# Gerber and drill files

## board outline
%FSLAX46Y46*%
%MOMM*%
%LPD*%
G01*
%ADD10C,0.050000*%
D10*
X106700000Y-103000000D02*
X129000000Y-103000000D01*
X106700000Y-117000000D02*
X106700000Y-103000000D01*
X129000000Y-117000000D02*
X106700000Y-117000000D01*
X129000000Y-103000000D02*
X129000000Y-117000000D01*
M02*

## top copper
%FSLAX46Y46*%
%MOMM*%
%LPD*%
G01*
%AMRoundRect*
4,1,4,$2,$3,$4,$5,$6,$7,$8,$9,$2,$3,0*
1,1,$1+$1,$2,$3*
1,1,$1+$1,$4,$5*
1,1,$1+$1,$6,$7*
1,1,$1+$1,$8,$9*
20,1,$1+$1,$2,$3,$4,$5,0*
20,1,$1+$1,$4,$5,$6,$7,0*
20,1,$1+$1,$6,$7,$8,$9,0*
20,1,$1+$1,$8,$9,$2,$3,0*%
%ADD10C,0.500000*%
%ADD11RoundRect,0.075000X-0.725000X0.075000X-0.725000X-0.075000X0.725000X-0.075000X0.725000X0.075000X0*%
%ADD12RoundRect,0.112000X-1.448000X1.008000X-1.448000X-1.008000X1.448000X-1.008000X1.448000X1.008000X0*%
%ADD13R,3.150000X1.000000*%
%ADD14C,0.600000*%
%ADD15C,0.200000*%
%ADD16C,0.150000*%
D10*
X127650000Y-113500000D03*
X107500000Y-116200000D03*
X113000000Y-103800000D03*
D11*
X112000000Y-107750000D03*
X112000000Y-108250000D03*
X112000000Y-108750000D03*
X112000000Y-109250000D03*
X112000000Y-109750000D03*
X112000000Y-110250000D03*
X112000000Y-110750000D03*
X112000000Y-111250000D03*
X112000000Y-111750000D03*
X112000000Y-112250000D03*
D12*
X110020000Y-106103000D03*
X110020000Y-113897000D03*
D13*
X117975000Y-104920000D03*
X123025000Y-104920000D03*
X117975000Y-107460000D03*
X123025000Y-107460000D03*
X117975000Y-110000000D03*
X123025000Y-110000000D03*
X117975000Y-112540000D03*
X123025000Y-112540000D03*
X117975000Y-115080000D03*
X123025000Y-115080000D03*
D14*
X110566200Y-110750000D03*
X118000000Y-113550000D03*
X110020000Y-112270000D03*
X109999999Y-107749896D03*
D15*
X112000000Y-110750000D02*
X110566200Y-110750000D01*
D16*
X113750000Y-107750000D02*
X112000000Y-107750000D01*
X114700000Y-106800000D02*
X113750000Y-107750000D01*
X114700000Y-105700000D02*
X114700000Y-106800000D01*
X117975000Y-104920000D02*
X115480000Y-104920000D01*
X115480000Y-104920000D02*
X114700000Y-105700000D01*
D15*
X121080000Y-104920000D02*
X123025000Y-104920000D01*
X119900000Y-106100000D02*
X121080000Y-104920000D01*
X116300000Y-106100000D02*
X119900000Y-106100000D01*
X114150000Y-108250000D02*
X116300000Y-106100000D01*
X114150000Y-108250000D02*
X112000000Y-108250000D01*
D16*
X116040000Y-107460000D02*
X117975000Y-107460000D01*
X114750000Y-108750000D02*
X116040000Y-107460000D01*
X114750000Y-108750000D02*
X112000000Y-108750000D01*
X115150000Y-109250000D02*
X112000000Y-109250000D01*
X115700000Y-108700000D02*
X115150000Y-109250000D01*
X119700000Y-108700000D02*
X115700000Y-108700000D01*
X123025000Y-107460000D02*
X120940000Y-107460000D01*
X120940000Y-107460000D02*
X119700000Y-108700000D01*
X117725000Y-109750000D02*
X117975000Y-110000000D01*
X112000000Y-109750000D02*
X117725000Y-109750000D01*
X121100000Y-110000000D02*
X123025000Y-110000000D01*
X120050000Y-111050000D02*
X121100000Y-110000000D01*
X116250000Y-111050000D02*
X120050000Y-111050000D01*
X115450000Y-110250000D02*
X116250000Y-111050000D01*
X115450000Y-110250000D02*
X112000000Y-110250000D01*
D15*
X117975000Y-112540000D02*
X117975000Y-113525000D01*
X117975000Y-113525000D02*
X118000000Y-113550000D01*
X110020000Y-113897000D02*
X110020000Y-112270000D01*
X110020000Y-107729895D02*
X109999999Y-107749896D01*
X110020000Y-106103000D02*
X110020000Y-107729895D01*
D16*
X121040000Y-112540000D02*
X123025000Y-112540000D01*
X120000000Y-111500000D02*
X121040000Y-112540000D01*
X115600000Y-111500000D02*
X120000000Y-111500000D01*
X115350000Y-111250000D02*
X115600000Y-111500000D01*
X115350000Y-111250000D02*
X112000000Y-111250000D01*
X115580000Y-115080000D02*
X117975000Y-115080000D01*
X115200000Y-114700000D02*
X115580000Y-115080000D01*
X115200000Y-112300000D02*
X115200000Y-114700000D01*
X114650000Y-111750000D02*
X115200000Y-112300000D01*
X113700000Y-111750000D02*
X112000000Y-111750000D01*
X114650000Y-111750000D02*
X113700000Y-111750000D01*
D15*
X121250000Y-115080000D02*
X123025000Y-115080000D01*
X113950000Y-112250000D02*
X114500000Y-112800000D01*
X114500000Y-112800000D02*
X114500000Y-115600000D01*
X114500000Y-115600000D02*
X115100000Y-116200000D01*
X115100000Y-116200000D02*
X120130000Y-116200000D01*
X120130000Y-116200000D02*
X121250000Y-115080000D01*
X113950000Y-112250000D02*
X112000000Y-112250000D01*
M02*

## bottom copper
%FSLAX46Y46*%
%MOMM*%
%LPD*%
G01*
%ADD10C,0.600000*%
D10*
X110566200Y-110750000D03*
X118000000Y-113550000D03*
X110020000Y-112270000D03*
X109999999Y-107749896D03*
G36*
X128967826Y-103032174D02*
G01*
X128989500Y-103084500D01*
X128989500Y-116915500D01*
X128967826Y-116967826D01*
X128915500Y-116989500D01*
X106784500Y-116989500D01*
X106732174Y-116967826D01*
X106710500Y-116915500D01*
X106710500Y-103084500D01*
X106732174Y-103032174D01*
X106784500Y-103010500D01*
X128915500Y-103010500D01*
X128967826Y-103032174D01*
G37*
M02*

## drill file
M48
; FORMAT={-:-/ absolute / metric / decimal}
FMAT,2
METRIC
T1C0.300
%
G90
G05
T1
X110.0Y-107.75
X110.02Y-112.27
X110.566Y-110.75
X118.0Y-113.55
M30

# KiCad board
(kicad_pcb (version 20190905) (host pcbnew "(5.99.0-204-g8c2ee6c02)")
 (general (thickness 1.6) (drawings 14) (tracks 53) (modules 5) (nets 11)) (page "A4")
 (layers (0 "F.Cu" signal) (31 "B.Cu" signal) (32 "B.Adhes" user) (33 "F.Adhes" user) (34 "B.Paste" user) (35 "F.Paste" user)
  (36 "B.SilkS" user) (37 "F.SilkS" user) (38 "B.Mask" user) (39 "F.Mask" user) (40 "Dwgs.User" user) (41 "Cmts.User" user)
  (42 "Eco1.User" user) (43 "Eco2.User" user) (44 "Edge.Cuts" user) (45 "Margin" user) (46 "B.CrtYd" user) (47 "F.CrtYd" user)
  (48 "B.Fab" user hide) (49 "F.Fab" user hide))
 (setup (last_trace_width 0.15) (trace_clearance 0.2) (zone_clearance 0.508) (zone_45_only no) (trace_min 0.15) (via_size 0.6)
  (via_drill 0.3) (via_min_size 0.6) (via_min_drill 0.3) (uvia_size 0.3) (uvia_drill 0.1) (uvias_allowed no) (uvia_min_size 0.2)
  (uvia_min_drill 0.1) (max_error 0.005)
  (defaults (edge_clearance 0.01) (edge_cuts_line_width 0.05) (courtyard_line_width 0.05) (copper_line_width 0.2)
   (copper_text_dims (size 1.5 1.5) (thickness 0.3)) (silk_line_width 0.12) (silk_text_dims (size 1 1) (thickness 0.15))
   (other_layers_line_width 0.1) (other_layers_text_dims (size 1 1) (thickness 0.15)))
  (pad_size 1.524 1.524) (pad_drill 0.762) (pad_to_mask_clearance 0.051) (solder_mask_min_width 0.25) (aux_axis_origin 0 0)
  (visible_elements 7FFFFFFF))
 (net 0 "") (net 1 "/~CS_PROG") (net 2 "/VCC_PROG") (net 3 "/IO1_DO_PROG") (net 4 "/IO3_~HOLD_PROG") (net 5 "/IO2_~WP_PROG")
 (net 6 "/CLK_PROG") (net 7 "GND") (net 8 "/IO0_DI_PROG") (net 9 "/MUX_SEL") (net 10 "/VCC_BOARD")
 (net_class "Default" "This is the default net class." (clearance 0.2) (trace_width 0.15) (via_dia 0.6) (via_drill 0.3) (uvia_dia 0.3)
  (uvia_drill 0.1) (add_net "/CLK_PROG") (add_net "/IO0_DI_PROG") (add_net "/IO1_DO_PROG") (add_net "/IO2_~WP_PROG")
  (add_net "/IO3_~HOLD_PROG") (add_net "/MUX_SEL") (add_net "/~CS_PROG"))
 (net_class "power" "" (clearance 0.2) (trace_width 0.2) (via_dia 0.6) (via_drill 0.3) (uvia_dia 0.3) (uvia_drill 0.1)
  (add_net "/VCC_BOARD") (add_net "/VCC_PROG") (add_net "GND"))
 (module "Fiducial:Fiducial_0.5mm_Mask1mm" (layer "F.Cu") (at 127.65 113.5)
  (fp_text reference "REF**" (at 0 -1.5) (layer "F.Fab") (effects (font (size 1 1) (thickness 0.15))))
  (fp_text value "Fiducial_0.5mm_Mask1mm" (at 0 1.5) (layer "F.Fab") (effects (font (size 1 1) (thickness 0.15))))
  (pad "" smd circle (at 0 0) (size 0.5 0.5) (layers "F.Cu" "F.Mask") (solder_mask_margin 0.25) (clearance 0.25)))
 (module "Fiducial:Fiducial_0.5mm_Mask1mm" (layer "F.Cu") (at 107.5 116.2)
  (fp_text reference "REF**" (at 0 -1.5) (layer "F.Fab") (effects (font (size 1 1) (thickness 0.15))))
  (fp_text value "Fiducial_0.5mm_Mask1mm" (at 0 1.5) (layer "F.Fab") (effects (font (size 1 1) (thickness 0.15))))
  (pad "" smd circle (at 0 0) (size 0.5 0.5) (layers "F.Cu" "F.Mask") (solder_mask_margin 0.25) (clearance 0.25)))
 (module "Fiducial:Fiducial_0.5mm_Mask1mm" (layer "F.Cu") (at 113 103.8)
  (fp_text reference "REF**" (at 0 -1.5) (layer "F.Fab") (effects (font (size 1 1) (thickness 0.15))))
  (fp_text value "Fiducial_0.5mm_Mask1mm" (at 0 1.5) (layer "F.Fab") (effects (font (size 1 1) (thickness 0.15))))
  (pad "" smd circle (at 0 0) (size 0.5 0.5) (layers "F.Cu" "F.Mask") (solder_mask_margin 0.25) (clearance 0.25)))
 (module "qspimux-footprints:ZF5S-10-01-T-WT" (layer "F.Cu") (at 112 110 -90)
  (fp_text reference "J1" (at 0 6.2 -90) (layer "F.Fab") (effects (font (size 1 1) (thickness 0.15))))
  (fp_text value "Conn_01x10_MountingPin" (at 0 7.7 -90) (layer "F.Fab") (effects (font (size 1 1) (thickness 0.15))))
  (pad "1" smd roundrect (at -2.25 0 270) (size 0.3 1.6) (layers "F.Cu" "F.Paste" "F.Mask") (roundrect_rratio 0.25) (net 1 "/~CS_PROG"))
  (pad "2" smd roundrect (at -1.75 0 270) (size 0.3 1.6) (layers "F.Cu" "F.Paste" "F.Mask") (roundrect_rratio 0.25) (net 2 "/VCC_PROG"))
  (pad "3" smd roundrect (at -1.25 0 270) (size 0.3 1.6) (layers "F.Cu" "F.Paste" "F.Mask") (roundrect_rratio 0.25) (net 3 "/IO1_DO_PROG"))
  (pad "4" smd roundrect (at -0.75 0 270) (size 0.3 1.6) (layers "F.Cu" "F.Paste" "F.Mask") (roundrect_rratio 0.25)
   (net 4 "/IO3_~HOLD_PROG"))
  (pad "5" smd roundrect (at -0.25 0 270) (size 0.3 1.6) (layers "F.Cu" "F.Paste" "F.Mask") (roundrect_rratio 0.25) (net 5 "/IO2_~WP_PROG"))
  (pad "6" smd roundrect (at 0.25 0 270) (size 0.3 1.6) (layers "F.Cu" "F.Paste" "F.Mask") (roundrect_rratio 0.25) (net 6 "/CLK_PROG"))
  (pad "7" smd roundrect (at 0.75 0 270) (size 0.3 1.6) (layers "F.Cu" "F.Paste" "F.Mask") (roundrect_rratio 0.25) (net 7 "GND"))
  (pad "8" smd roundrect (at 1.25 0 270) (size 0.3 1.6) (layers "F.Cu" "F.Paste" "F.Mask") (roundrect_rratio 0.25) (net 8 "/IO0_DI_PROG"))
  (pad "9" smd roundrect (at 1.75 0 270) (size 0.3 1.6) (layers "F.Cu" "F.Paste" "F.Mask") (roundrect_rratio 0.25) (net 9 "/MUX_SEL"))
  (pad "10" smd roundrect (at 2.25 0 270) (size 0.3 1.6) (layers "F.Cu" "F.Paste" "F.Mask") (roundrect_rratio 0.25) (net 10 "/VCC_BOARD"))
  (pad "MP" smd roundrect (at -3.897 1.98 270) (size 2.24 3.12) (layers "F.Cu" "F.Paste" "F.Mask") (roundrect_rratio 0.05) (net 7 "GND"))
  (pad "MP" smd roundrect (at 3.897 1.98 270) (size 2.24 3.12) (layers "F.Cu" "F.Paste" "F.Mask") (roundrect_rratio 0.05) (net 7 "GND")))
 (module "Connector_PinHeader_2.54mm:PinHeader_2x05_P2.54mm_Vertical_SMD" (layer "F.Cu") (at 120.5 110)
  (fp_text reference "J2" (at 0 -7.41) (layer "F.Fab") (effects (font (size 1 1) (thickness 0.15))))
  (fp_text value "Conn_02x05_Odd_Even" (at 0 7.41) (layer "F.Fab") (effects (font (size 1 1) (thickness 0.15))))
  (pad "1" smd rect (at -2.525 -5.08) (size 3.15 1) (layers "F.Cu" "F.Paste" "F.Mask") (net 1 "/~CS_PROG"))
  (pad "2" smd rect (at 2.525 -5.08) (size 3.15 1) (layers "F.Cu" "F.Paste" "F.Mask") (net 2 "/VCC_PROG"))
  (pad "3" smd rect (at -2.525 -2.54) (size 3.15 1) (layers "F.Cu" "F.Paste" "F.Mask") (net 3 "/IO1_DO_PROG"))
  (pad "4" smd rect (at 2.525 -2.54) (size 3.15 1) (layers "F.Cu" "F.Paste" "F.Mask") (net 4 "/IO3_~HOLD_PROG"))
  (pad "5" smd rect (at -2.525 0) (size 3.15 1) (layers "F.Cu" "F.Paste" "F.Mask") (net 5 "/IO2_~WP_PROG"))
  (pad "6" smd rect (at 2.525 0) (size 3.15 1) (layers "F.Cu" "F.Paste" "F.Mask") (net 6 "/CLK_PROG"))
  (pad "7" smd rect (at -2.525 2.54) (size 3.15 1) (layers "F.Cu" "F.Paste" "F.Mask") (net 7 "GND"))
  (pad "8" smd rect (at 2.525 2.54) (size 3.15 1) (layers "F.Cu" "F.Paste" "F.Mask") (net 8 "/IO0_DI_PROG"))
  (pad "9" smd rect (at -2.525 5.08) (size 3.15 1) (layers "F.Cu" "F.Paste" "F.Mask") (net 9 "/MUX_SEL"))
  (pad "10" smd rect (at 2.525 5.08) (size 3.15 1) (layers "F.Cu" "F.Paste" "F.Mask") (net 10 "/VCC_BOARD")))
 (gr_line (start 106.7 103) (end 129 103) (layer "Edge.Cuts") (width 0.05))
 (gr_line (start 106.7 117) (end 106.7 103) (layer "Edge.Cuts") (width 0.05))
 (gr_line (start 129 117) (end 106.7 117) (layer "Edge.Cuts") (width 0.05))
 (gr_line (start 129 103) (end 129 117) (layer "Edge.Cuts") (width 0.05))
 (segment (start 112 110.75) (end 110.5662 110.75) (width 0.2) (layer "F.Cu") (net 7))
 (via (at 110.5662 110.75) (size 0.6) (drill 0.3) (layers "F.Cu" "B.Cu") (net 7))
 (segment (start 113.75 107.75) (end 112 107.75) (width 0.15) (layer "F.Cu") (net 1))
 (segment (start 114.7 106.8) (end 113.75 107.75) (width 0.15) (layer "F.Cu") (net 1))
 (segment (start 114.7 105.7) (end 114.7 106.8) (width 0.15) (layer "F.Cu") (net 1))
 (segment (start 117.975 104.92) (end 115.48 104.92) (width 0.15) (layer "F.Cu") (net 1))
 (segment (start 115.48 104.92) (end 114.7 105.7) (width 0.15) (layer "F.Cu") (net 1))
 (segment (start 121.08 104.92) (end 123.025 104.92) (width 0.2) (layer "F.Cu") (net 2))
 (segment (start 119.9 106.1) (end 121.08 104.92) (width 0.2) (layer "F.Cu") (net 2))
 (segment (start 116.3 106.1) (end 119.9 106.1) (width 0.2) (layer "F.Cu") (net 2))
 (segment (start 114.15 108.25) (end 116.3 106.1) (width 0.2) (layer "F.Cu") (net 2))
 (segment (start 114.15 108.25) (end 112 108.25) (width 0.2) (layer "F.Cu") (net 2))
 (segment (start 116.04 107.46) (end 117.975 107.46) (width 0.15) (layer "F.Cu") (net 3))
 (segment (start 114.75 108.75) (end 116.04 107.46) (width 0.15) (layer "F.Cu") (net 3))
 (segment (start 114.75 108.75) (end 112 108.75) (width 0.15) (layer "F.Cu") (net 3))
 (segment (start 115.15 109.25) (end 112 109.25) (width 0.15) (layer "F.Cu") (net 4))
 (segment (start 115.7 108.7) (end 115.15 109.25) (width 0.15) (layer "F.Cu") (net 4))
 (segment (start 119.7 108.7) (end 115.7 108.7) (width 0.15) (layer "F.Cu") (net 4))
 (segment (start 123.025 107.46) (end 120.94 107.46) (width 0.15) (layer "F.Cu") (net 4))
 (segment (start 120.94 107.46) (end 119.7 108.7) (width 0.15) (layer "F.Cu") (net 4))
 (segment (start 117.725 109.75) (end 117.975 110) (width 0.15) (layer "F.Cu") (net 5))
 (segment (start 112 109.75) (end 117.725 109.75) (width 0.15) (layer "F.Cu") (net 5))
 (segment (start 121.1 110) (end 123.025 110) (width 0.15) (layer "F.Cu") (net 6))
 (segment (start 120.05 111.05) (end 121.1 110) (width 0.15) (layer "F.Cu") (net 6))
 (segment (start 116.25 111.05) (end 120.05 111.05) (width 0.15) (layer "F.Cu") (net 6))
 (segment (start 115.45 110.25) (end 116.25 111.05) (width 0.15) (layer "F.Cu") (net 6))
 (segment (start 115.45 110.25) (end 112 110.25) (width 0.15) (layer "F.Cu") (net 6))
 (via (at 118 113.55) (size 0.6) (drill 0.3) (layers "F.Cu" "B.Cu") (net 7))
 (segment (start 117.975 112.54) (end 117.975 113.525) (width 0.2) (layer "F.Cu") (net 7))
 (segment (start 117.975 113.525) (end 118 113.55) (width 0.2) (layer "F.Cu") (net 7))
 (segment (start 110.02 113.897) (end 110.02 112.27) (width 0.2) (layer "F.Cu") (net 7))
 (via (at 110.02 112.27) (size 0.6) (drill 0.3) (layers "F.Cu" "B.Cu") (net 7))
 (via (at 109.999999 107.749896) (size 0.6) (drill 0.3) (layers "F.Cu" "B.Cu") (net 7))
 (segment (start 110.02 107.729895) (end 109.999999 107.749896) (width 0.2) (layer "F.Cu") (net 7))
 (segment (start 110.02 106.103) (end 110.02 107.729895) (width 0.2) (layer "F.Cu") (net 7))
 (segment (start 121.04 112.54) (end 123.025 112.54) (width 0.15) (layer "F.Cu") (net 8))
 (segment (start 120 111.5) (end 121.04 112.54) (width 0.15) (layer "F.Cu") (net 8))
 (segment (start 115.6 111.5) (end 120 111.5) (width 0.15) (layer "F.Cu") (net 8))
 (segment (start 115.35 111.25) (end 115.6 111.5) (width 0.15) (layer "F.Cu") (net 8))
 (segment (start 115.35 111.25) (end 112 111.25) (width 0.15) (layer "F.Cu") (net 8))
 (segment (start 115.58 115.08) (end 117.975 115.08) (width 0.15) (layer "F.Cu") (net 9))
 (segment (start 115.2 114.7) (end 115.58 115.08) (width 0.15) (layer "F.Cu") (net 9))
 (segment (start 115.2 112.3) (end 115.2 114.7) (width 0.15) (layer "F.Cu") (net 9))
 (segment (start 114.65 111.75) (end 115.2 112.3) (width 0.15) (layer "F.Cu") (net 9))
 (segment (start 113.7 111.75) (end 112 111.75) (width 0.15) (layer "F.Cu") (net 9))
 (segment (start 114.65 111.75) (end 113.7 111.75) (width 0.15) (layer "F.Cu") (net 9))
 (segment (start 121.25 115.08) (end 123.025 115.08) (width 0.2) (layer "F.Cu") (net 10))
 (segment (start 113.95 112.25) (end 114.5 112.8) (width 0.2) (layer "F.Cu") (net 10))
 (segment (start 114.5 112.8) (end 114.5 115.6) (width 0.2) (layer "F.Cu") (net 10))
 (segment (start 114.5 115.6) (end 115.1 116.2) (width 0.2) (layer "F.Cu") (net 10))
 (segment (start 115.1 116.2) (end 120.13 116.2) (width 0.2) (layer "F.Cu") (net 10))
 (segment (start 120.13 116.2) (end 121.25 115.08) (width 0.2) (layer "F.Cu") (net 10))
 (segment (start 113.95 112.25) (end 112 112.25) (width 0.2) (layer "F.Cu") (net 10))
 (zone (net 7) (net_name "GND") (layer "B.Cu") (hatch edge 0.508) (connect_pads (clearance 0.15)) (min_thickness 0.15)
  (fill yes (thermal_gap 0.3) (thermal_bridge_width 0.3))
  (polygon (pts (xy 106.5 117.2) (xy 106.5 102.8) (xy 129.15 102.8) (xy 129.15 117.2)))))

